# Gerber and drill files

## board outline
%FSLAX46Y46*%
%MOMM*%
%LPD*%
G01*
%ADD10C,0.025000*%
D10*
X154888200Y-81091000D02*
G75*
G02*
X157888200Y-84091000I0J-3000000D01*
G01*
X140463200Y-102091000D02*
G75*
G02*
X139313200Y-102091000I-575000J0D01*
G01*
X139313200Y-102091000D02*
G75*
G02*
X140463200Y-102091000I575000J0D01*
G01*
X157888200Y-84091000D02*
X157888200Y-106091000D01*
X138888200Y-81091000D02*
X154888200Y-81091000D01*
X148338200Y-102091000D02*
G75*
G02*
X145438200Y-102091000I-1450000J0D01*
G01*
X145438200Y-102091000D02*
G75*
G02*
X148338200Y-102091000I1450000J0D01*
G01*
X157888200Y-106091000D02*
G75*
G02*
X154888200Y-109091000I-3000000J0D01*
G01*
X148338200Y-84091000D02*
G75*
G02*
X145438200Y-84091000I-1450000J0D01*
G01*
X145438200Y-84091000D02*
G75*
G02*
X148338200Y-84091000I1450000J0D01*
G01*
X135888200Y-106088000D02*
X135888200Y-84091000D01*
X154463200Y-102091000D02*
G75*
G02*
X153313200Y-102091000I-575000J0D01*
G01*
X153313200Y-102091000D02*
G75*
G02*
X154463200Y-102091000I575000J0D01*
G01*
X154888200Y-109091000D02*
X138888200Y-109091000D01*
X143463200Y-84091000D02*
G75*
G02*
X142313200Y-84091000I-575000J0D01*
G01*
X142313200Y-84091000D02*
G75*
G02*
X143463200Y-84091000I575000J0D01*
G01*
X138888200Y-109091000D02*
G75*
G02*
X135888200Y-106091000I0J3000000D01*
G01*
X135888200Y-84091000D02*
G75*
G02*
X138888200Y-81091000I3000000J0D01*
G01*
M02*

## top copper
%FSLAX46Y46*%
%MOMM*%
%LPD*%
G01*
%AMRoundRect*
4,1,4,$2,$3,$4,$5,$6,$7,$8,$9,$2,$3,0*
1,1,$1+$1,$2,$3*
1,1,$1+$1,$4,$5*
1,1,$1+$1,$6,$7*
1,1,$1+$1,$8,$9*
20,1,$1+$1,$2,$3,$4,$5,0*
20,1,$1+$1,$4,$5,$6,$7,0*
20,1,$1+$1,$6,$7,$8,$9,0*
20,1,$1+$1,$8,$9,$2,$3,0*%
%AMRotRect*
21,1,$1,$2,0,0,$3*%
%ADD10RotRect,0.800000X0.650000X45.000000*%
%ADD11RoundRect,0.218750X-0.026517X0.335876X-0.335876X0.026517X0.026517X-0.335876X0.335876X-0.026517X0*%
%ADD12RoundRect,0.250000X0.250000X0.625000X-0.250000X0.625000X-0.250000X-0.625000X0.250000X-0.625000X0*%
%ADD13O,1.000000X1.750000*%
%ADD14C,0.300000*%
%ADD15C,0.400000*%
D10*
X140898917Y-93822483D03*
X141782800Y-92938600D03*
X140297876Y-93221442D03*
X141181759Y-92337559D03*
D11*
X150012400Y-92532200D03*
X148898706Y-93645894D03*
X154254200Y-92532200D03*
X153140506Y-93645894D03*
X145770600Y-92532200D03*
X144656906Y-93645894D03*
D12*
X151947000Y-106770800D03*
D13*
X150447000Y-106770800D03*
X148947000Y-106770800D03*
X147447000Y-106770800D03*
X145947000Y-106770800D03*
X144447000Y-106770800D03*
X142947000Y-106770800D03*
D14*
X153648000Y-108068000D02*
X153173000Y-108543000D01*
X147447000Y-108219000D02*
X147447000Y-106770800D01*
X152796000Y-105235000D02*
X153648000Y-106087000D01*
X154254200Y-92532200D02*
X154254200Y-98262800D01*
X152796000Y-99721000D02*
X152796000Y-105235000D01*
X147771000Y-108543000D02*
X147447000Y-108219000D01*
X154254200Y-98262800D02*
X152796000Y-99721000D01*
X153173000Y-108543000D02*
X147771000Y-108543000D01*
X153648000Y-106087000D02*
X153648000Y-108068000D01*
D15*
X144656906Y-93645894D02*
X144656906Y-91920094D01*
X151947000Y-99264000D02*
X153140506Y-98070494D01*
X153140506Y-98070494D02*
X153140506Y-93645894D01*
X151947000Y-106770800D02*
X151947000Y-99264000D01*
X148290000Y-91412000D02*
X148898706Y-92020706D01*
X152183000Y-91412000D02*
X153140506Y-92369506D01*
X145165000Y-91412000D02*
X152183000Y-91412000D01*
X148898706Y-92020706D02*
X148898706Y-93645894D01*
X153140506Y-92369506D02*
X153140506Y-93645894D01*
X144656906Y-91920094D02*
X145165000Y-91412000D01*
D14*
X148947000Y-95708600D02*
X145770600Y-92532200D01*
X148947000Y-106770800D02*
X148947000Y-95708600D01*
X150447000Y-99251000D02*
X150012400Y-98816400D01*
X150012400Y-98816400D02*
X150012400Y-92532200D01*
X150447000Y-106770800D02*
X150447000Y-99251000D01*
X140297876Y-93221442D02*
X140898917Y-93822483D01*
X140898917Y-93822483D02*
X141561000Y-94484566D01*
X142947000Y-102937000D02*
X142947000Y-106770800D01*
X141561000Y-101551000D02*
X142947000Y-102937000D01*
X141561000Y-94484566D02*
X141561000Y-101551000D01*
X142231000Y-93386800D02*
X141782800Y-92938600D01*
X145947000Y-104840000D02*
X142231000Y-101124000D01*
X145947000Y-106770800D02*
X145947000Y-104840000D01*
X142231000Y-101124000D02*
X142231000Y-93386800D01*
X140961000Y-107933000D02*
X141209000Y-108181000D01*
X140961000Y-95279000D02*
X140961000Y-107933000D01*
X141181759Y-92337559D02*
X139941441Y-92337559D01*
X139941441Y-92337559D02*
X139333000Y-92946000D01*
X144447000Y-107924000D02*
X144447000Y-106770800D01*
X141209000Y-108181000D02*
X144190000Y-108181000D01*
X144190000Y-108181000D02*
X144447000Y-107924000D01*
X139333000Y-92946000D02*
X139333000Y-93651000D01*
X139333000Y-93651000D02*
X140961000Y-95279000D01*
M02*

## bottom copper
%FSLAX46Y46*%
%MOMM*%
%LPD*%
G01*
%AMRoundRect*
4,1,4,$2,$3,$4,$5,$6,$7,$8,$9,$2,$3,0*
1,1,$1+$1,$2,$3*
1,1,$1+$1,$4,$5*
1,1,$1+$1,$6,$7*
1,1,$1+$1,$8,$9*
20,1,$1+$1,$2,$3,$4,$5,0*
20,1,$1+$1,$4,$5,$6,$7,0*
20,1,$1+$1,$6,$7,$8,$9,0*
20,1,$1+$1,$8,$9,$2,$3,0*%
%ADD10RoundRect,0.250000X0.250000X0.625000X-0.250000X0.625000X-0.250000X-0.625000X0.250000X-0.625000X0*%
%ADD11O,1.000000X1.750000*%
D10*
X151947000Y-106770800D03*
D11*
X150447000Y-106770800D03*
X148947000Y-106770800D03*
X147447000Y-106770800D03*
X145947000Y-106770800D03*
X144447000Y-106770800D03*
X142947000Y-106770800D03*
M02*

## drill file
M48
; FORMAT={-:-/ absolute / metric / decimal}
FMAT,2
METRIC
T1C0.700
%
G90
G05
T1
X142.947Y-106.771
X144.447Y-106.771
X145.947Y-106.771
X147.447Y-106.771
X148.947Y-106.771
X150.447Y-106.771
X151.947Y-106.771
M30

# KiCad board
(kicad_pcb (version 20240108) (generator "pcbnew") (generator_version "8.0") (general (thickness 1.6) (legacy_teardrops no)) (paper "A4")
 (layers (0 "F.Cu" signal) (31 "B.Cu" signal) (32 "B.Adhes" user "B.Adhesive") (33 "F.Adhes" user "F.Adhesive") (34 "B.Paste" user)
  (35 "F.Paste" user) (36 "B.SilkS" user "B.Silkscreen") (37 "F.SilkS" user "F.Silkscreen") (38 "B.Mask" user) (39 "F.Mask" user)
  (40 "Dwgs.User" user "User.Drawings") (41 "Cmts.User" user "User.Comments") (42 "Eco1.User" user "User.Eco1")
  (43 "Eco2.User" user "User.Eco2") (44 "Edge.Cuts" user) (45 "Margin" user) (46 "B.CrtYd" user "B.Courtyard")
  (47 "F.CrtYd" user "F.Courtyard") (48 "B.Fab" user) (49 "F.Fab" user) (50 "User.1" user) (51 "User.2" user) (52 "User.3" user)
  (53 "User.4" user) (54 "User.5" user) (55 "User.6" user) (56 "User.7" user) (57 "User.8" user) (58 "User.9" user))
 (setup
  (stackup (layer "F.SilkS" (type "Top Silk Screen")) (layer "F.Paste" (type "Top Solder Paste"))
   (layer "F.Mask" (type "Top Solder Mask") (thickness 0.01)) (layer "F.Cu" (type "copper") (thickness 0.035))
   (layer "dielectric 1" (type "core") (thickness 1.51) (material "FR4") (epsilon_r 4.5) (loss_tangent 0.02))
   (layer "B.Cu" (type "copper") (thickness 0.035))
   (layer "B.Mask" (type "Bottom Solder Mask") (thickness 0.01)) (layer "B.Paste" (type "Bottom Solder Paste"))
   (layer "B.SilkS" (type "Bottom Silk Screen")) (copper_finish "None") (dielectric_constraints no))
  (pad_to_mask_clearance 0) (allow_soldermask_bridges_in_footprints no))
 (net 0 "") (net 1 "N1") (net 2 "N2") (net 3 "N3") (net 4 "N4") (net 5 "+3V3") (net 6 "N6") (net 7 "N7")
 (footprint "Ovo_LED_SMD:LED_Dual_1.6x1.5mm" (layer "F.Cu") (at 141.040338 93.080021 45)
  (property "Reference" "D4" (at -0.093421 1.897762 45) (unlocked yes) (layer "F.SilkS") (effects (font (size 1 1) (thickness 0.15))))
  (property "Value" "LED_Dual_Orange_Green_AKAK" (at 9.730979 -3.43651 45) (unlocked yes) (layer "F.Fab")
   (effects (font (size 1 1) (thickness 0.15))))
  (pad "1" smd rect (at -0.625 0.425 45) (size 0.8 0.65) (layers "F.Cu" "F.Paste" "F.Mask") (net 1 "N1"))
  (pad "2" smd rect (at 0.625 0.425 45) (size 0.8 0.65) (layers "F.Cu" "F.Paste" "F.Mask") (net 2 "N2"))
  (pad "3" smd rect (at -0.625 -0.425 45) (size 0.8 0.65) (layers "F.Cu" "F.Paste" "F.Mask") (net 1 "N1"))
  (pad "4" smd rect (at 0.625 -0.425 45) (size 0.8 0.65) (layers "F.Cu" "F.Paste" "F.Mask") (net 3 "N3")))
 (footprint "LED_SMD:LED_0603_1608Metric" (layer "F.Cu") (at 149.455553 93.089047 -135)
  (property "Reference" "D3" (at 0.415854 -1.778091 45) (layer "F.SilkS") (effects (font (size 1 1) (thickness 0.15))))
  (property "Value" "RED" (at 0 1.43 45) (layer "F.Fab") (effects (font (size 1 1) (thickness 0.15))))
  (pad "1" smd roundrect (at -0.787501 0 225) (size 0.875 0.95) (layers "F.Cu" "F.Paste" "F.Mask") (roundrect_rratio 0.25) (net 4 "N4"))
  (pad "2" smd roundrect (at 0.787501 0 225) (size 0.875 0.95) (layers "F.Cu" "F.Paste" "F.Mask") (roundrect_rratio 0.25) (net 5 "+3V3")))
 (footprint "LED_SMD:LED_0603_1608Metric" (layer "F.Cu") (at 153.697353 93.089047 -135)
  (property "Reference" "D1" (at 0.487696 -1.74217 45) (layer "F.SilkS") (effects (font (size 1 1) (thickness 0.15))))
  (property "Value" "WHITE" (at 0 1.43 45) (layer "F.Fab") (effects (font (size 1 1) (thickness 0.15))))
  (pad "1" smd roundrect (at -0.787501 0 225) (size 0.875 0.95) (layers "F.Cu" "F.Paste" "F.Mask") (roundrect_rratio 0.25) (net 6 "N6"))
  (pad "2" smd roundrect (at 0.787501 0 225) (size 0.875 0.95) (layers "F.Cu" "F.Paste" "F.Mask") (roundrect_rratio 0.25) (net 5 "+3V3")))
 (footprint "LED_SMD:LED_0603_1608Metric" (layer "F.Cu") (at 145.213753 93.089047 -135)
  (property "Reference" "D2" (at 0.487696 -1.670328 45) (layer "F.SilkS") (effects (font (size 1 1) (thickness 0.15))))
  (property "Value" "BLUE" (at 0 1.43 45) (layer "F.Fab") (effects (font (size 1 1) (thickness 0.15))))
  (pad "1" smd roundrect (at -0.787501 0 225) (size 0.875 0.95) (layers "F.Cu" "F.Paste" "F.Mask") (roundrect_rratio 0.25) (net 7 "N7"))
  (pad "2" smd roundrect (at 0.787501 0 225) (size 0.875 0.95) (layers "F.Cu" "F.Paste" "F.Mask") (roundrect_rratio 0.25) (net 5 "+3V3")))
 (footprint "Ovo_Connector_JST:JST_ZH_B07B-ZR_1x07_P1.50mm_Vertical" (layer "B.Cu") (at 151.947 106.7708 180)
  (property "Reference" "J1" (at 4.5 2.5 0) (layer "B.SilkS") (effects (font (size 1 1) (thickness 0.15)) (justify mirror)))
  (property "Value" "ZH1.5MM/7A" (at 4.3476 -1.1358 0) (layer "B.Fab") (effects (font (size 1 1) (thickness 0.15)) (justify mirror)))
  (pad "1" thru_hole roundrect (at 0 0 180) (size 1 1.75) (drill 0.7) (layers "*.Cu" "*.Mask") (remove_unused_layers no)
   (roundrect_rratio 0.25) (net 5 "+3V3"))
  (pad "2" thru_hole oval (at 1.5 0 180) (size 1 1.75) (drill 0.7) (layers "*.Cu" "*.Mask") (remove_unused_layers no) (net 4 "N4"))
  (pad "3" thru_hole oval (at 3 0 180) (size 1 1.75) (drill 0.7) (layers "*.Cu" "*.Mask") (remove_unused_layers no) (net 7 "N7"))
  (pad "4" thru_hole oval (at 4.5 0 180) (size 1 1.75) (drill 0.7) (layers "*.Cu" "*.Mask") (remove_unused_layers no) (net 6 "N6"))
  (pad "5" thru_hole oval (at 6 0 180) (size 1 1.75) (drill 0.7) (layers "*.Cu" "*.Mask") (remove_unused_layers no) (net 2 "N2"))
  (pad "6" thru_hole oval (at 7.5 0 180) (size 1 1.75) (drill 0.7) (layers "*.Cu" "*.Mask") (remove_unused_layers no) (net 3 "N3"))
  (pad "7" thru_hole oval (at 9 0 180) (size 1 1.75) (drill 0.7) (layers "*.Cu" "*.Mask") (remove_unused_layers no) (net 1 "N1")))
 (gr_arc (start 154.8882 81.091) (mid 157.009521 81.96968) (end 157.8882 84.091) (stroke (width 0.025) (type solid)) (layer "Edge.Cuts"))
 (gr_circle (center 139.8882 102.091) (end 140.4632 102.091) (stroke (width 0.025) (type solid)) (fill none) (layer "Edge.Cuts"))
 (gr_line (start 157.8882 84.091) (end 157.8882 106.091) (stroke (width 0.025) (type solid)) (layer "Edge.Cuts"))
 (gr_line (start 138.8882 81.091) (end 154.8882 81.091) (stroke (width 0.025) (type solid)) (layer "Edge.Cuts"))
 (gr_circle (center 146.8882 102.091) (end 148.3382 102.091) (stroke (width 0.025) (type solid)) (fill none) (layer "Edge.Cuts"))
 (gr_arc (start 157.8882 106.091) (mid 157.00952 108.21232) (end 154.8882 109.091) (stroke (width 0.025) (type solid)) (layer "Edge.Cuts"))
 (gr_circle (center 146.8882 84.091) (end 148.3382 84.091) (stroke (width 0.025) (type solid)) (fill none) (layer "Edge.Cuts"))
 (gr_line (start 135.8882 106.088) (end 135.8882 84.091) (stroke (width 0.025) (type solid)) (layer "Edge.Cuts"))
 (gr_circle (center 153.8882 102.091) (end 154.4632 102.091) (stroke (width 0.025) (type solid)) (fill none) (layer "Edge.Cuts"))
 (gr_line (start 154.8882 109.091) (end 138.8882 109.091) (stroke (width 0.025) (type solid)) (layer "Edge.Cuts"))
 (gr_circle (center 142.8882 84.091) (end 143.4632 84.091) (stroke (width 0.025) (type solid)) (fill none) (layer "Edge.Cuts"))
 (gr_arc (start 138.8882 109.091) (mid 136.76688 108.21232) (end 135.8882 106.091) (stroke (width 0.025) (type solid)) (layer "Edge.Cuts"))
 (gr_arc (start 135.8882 84.091) (mid 136.766878 81.969678) (end 138.8882 81.091) (stroke (width 0.025) (type solid)) (layer "Edge.Cuts"))
 (segment (start 153.648 108.068) (end 153.173 108.543) (width 0.3) (layer "F.Cu") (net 6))
 (segment (start 147.447 108.219) (end 147.447 106.7708) (width 0.3) (layer "F.Cu") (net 6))
 (segment (start 152.796 105.235) (end 153.648 106.087) (width 0.3) (layer "F.Cu") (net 6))
 (segment (start 154.2542 92.5322) (end 154.2542 98.2628) (width 0.3) (layer "F.Cu") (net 6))
 (segment (start 152.796 99.721) (end 152.796 105.235) (width 0.3) (layer "F.Cu") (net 6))
 (segment (start 147.771 108.543) (end 147.447 108.219) (width 0.3) (layer "F.Cu") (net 6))
 (segment (start 154.2542 98.2628) (end 152.796 99.721) (width 0.3) (layer "F.Cu") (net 6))
 (segment (start 153.173 108.543) (end 147.771 108.543) (width 0.3) (layer "F.Cu") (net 6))
 (segment (start 153.648 106.087) (end 153.648 108.068) (width 0.3) (layer "F.Cu") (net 6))
 (segment (start 144.656906 93.645894) (end 144.656906 91.920094) (width 0.4) (layer "F.Cu") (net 5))
 (segment (start 151.947 99.264) (end 153.140506 98.070494) (width 0.4) (layer "F.Cu") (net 5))
 (segment (start 153.140506 98.070494) (end 153.140506 93.645894) (width 0.4) (layer "F.Cu") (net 5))
 (segment (start 151.947 106.7708) (end 151.947 99.264) (width 0.4) (layer "F.Cu") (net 5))
 (segment (start 148.29 91.412) (end 148.898706 92.020706) (width 0.4) (layer "F.Cu") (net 5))
 (segment (start 152.183 91.412) (end 153.140506 92.369506) (width 0.4) (layer "F.Cu") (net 5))
 (segment (start 145.165 91.412) (end 152.183 91.412) (width 0.4) (layer "F.Cu") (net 5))
 (segment (start 148.898706 92.020706) (end 148.898706 93.645894) (width 0.4) (layer "F.Cu") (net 5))
 (segment (start 153.140506 92.369506) (end 153.140506 93.645894) (width 0.4) (layer "F.Cu") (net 5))
 (segment (start 144.656906 91.920094) (end 145.165 91.412) (width 0.4) (layer "F.Cu") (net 5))
 (segment (start 148.947 95.7086) (end 145.7706 92.5322) (width 0.3) (layer "F.Cu") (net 7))
 (segment (start 148.947 106.7708) (end 148.947 95.7086) (width 0.3) (layer "F.Cu") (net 7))
 (segment (start 150.447 99.251) (end 150.0124 98.8164) (width 0.3) (layer "F.Cu") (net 4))
 (segment (start 150.0124 98.8164) (end 150.0124 92.5322) (width 0.3) (layer "F.Cu") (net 4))
 (segment (start 150.447 106.7708) (end 150.447 99.251) (width 0.3) (layer "F.Cu") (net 4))
 (segment (start 140.297876 93.221442) (end 140.898917 93.822483) (width 0.3) (layer "F.Cu") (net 1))
 (segment (start 140.898917 93.822483) (end 141.561 94.484566) (width 0.3) (layer "F.Cu") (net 1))
 (segment (start 142.947 102.937) (end 142.947 106.7708) (width 0.3) (layer "F.Cu") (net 1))
 (segment (start 141.561 101.551) (end 142.947 102.937) (width 0.3) (layer "F.Cu") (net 1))
 (segment (start 141.561 94.484566) (end 141.561 101.551) (width 0.3) (layer "F.Cu") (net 1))
 (segment (start 142.231 93.3868) (end 141.7828 92.9386) (width 0.3) (layer "F.Cu") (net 2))
 (segment (start 145.947 104.84) (end 142.231 101.124) (width 0.3) (layer "F.Cu") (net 2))
 (segment (start 145.947 106.7708) (end 145.947 104.84) (width 0.3) (layer "F.Cu") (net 2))
 (segment (start 142.231 101.124) (end 142.231 93.3868) (width 0.3) (layer "F.Cu") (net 2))
 (segment (start 140.961 107.933) (end 141.209 108.181) (width 0.3) (layer "F.Cu") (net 3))
 (segment (start 140.961 95.279) (end 140.961 107.933) (width 0.3) (layer "F.Cu") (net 3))
 (segment (start 141.181759 92.337559) (end 139.941441 92.337559) (width 0.3) (layer "F.Cu") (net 3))
 (segment (start 139.941441 92.337559) (end 139.333 92.946) (width 0.3) (layer "F.Cu") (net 3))
 (segment (start 144.447 107.924) (end 144.447 106.7708) (width 0.3) (layer "F.Cu") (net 3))
 (segment (start 141.209 108.181) (end 144.19 108.181) (width 0.3) (layer "F.Cu") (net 3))
 (segment (start 144.19 108.181) (end 144.447 107.924) (width 0.3) (layer "F.Cu") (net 3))
 (segment (start 139.333 92.946) (end 139.333 93.651) (width 0.3) (layer "F.Cu") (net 3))
 (segment (start 139.333 93.651) (end 140.961 95.279) (width 0.3) (layer "F.Cu") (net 3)))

